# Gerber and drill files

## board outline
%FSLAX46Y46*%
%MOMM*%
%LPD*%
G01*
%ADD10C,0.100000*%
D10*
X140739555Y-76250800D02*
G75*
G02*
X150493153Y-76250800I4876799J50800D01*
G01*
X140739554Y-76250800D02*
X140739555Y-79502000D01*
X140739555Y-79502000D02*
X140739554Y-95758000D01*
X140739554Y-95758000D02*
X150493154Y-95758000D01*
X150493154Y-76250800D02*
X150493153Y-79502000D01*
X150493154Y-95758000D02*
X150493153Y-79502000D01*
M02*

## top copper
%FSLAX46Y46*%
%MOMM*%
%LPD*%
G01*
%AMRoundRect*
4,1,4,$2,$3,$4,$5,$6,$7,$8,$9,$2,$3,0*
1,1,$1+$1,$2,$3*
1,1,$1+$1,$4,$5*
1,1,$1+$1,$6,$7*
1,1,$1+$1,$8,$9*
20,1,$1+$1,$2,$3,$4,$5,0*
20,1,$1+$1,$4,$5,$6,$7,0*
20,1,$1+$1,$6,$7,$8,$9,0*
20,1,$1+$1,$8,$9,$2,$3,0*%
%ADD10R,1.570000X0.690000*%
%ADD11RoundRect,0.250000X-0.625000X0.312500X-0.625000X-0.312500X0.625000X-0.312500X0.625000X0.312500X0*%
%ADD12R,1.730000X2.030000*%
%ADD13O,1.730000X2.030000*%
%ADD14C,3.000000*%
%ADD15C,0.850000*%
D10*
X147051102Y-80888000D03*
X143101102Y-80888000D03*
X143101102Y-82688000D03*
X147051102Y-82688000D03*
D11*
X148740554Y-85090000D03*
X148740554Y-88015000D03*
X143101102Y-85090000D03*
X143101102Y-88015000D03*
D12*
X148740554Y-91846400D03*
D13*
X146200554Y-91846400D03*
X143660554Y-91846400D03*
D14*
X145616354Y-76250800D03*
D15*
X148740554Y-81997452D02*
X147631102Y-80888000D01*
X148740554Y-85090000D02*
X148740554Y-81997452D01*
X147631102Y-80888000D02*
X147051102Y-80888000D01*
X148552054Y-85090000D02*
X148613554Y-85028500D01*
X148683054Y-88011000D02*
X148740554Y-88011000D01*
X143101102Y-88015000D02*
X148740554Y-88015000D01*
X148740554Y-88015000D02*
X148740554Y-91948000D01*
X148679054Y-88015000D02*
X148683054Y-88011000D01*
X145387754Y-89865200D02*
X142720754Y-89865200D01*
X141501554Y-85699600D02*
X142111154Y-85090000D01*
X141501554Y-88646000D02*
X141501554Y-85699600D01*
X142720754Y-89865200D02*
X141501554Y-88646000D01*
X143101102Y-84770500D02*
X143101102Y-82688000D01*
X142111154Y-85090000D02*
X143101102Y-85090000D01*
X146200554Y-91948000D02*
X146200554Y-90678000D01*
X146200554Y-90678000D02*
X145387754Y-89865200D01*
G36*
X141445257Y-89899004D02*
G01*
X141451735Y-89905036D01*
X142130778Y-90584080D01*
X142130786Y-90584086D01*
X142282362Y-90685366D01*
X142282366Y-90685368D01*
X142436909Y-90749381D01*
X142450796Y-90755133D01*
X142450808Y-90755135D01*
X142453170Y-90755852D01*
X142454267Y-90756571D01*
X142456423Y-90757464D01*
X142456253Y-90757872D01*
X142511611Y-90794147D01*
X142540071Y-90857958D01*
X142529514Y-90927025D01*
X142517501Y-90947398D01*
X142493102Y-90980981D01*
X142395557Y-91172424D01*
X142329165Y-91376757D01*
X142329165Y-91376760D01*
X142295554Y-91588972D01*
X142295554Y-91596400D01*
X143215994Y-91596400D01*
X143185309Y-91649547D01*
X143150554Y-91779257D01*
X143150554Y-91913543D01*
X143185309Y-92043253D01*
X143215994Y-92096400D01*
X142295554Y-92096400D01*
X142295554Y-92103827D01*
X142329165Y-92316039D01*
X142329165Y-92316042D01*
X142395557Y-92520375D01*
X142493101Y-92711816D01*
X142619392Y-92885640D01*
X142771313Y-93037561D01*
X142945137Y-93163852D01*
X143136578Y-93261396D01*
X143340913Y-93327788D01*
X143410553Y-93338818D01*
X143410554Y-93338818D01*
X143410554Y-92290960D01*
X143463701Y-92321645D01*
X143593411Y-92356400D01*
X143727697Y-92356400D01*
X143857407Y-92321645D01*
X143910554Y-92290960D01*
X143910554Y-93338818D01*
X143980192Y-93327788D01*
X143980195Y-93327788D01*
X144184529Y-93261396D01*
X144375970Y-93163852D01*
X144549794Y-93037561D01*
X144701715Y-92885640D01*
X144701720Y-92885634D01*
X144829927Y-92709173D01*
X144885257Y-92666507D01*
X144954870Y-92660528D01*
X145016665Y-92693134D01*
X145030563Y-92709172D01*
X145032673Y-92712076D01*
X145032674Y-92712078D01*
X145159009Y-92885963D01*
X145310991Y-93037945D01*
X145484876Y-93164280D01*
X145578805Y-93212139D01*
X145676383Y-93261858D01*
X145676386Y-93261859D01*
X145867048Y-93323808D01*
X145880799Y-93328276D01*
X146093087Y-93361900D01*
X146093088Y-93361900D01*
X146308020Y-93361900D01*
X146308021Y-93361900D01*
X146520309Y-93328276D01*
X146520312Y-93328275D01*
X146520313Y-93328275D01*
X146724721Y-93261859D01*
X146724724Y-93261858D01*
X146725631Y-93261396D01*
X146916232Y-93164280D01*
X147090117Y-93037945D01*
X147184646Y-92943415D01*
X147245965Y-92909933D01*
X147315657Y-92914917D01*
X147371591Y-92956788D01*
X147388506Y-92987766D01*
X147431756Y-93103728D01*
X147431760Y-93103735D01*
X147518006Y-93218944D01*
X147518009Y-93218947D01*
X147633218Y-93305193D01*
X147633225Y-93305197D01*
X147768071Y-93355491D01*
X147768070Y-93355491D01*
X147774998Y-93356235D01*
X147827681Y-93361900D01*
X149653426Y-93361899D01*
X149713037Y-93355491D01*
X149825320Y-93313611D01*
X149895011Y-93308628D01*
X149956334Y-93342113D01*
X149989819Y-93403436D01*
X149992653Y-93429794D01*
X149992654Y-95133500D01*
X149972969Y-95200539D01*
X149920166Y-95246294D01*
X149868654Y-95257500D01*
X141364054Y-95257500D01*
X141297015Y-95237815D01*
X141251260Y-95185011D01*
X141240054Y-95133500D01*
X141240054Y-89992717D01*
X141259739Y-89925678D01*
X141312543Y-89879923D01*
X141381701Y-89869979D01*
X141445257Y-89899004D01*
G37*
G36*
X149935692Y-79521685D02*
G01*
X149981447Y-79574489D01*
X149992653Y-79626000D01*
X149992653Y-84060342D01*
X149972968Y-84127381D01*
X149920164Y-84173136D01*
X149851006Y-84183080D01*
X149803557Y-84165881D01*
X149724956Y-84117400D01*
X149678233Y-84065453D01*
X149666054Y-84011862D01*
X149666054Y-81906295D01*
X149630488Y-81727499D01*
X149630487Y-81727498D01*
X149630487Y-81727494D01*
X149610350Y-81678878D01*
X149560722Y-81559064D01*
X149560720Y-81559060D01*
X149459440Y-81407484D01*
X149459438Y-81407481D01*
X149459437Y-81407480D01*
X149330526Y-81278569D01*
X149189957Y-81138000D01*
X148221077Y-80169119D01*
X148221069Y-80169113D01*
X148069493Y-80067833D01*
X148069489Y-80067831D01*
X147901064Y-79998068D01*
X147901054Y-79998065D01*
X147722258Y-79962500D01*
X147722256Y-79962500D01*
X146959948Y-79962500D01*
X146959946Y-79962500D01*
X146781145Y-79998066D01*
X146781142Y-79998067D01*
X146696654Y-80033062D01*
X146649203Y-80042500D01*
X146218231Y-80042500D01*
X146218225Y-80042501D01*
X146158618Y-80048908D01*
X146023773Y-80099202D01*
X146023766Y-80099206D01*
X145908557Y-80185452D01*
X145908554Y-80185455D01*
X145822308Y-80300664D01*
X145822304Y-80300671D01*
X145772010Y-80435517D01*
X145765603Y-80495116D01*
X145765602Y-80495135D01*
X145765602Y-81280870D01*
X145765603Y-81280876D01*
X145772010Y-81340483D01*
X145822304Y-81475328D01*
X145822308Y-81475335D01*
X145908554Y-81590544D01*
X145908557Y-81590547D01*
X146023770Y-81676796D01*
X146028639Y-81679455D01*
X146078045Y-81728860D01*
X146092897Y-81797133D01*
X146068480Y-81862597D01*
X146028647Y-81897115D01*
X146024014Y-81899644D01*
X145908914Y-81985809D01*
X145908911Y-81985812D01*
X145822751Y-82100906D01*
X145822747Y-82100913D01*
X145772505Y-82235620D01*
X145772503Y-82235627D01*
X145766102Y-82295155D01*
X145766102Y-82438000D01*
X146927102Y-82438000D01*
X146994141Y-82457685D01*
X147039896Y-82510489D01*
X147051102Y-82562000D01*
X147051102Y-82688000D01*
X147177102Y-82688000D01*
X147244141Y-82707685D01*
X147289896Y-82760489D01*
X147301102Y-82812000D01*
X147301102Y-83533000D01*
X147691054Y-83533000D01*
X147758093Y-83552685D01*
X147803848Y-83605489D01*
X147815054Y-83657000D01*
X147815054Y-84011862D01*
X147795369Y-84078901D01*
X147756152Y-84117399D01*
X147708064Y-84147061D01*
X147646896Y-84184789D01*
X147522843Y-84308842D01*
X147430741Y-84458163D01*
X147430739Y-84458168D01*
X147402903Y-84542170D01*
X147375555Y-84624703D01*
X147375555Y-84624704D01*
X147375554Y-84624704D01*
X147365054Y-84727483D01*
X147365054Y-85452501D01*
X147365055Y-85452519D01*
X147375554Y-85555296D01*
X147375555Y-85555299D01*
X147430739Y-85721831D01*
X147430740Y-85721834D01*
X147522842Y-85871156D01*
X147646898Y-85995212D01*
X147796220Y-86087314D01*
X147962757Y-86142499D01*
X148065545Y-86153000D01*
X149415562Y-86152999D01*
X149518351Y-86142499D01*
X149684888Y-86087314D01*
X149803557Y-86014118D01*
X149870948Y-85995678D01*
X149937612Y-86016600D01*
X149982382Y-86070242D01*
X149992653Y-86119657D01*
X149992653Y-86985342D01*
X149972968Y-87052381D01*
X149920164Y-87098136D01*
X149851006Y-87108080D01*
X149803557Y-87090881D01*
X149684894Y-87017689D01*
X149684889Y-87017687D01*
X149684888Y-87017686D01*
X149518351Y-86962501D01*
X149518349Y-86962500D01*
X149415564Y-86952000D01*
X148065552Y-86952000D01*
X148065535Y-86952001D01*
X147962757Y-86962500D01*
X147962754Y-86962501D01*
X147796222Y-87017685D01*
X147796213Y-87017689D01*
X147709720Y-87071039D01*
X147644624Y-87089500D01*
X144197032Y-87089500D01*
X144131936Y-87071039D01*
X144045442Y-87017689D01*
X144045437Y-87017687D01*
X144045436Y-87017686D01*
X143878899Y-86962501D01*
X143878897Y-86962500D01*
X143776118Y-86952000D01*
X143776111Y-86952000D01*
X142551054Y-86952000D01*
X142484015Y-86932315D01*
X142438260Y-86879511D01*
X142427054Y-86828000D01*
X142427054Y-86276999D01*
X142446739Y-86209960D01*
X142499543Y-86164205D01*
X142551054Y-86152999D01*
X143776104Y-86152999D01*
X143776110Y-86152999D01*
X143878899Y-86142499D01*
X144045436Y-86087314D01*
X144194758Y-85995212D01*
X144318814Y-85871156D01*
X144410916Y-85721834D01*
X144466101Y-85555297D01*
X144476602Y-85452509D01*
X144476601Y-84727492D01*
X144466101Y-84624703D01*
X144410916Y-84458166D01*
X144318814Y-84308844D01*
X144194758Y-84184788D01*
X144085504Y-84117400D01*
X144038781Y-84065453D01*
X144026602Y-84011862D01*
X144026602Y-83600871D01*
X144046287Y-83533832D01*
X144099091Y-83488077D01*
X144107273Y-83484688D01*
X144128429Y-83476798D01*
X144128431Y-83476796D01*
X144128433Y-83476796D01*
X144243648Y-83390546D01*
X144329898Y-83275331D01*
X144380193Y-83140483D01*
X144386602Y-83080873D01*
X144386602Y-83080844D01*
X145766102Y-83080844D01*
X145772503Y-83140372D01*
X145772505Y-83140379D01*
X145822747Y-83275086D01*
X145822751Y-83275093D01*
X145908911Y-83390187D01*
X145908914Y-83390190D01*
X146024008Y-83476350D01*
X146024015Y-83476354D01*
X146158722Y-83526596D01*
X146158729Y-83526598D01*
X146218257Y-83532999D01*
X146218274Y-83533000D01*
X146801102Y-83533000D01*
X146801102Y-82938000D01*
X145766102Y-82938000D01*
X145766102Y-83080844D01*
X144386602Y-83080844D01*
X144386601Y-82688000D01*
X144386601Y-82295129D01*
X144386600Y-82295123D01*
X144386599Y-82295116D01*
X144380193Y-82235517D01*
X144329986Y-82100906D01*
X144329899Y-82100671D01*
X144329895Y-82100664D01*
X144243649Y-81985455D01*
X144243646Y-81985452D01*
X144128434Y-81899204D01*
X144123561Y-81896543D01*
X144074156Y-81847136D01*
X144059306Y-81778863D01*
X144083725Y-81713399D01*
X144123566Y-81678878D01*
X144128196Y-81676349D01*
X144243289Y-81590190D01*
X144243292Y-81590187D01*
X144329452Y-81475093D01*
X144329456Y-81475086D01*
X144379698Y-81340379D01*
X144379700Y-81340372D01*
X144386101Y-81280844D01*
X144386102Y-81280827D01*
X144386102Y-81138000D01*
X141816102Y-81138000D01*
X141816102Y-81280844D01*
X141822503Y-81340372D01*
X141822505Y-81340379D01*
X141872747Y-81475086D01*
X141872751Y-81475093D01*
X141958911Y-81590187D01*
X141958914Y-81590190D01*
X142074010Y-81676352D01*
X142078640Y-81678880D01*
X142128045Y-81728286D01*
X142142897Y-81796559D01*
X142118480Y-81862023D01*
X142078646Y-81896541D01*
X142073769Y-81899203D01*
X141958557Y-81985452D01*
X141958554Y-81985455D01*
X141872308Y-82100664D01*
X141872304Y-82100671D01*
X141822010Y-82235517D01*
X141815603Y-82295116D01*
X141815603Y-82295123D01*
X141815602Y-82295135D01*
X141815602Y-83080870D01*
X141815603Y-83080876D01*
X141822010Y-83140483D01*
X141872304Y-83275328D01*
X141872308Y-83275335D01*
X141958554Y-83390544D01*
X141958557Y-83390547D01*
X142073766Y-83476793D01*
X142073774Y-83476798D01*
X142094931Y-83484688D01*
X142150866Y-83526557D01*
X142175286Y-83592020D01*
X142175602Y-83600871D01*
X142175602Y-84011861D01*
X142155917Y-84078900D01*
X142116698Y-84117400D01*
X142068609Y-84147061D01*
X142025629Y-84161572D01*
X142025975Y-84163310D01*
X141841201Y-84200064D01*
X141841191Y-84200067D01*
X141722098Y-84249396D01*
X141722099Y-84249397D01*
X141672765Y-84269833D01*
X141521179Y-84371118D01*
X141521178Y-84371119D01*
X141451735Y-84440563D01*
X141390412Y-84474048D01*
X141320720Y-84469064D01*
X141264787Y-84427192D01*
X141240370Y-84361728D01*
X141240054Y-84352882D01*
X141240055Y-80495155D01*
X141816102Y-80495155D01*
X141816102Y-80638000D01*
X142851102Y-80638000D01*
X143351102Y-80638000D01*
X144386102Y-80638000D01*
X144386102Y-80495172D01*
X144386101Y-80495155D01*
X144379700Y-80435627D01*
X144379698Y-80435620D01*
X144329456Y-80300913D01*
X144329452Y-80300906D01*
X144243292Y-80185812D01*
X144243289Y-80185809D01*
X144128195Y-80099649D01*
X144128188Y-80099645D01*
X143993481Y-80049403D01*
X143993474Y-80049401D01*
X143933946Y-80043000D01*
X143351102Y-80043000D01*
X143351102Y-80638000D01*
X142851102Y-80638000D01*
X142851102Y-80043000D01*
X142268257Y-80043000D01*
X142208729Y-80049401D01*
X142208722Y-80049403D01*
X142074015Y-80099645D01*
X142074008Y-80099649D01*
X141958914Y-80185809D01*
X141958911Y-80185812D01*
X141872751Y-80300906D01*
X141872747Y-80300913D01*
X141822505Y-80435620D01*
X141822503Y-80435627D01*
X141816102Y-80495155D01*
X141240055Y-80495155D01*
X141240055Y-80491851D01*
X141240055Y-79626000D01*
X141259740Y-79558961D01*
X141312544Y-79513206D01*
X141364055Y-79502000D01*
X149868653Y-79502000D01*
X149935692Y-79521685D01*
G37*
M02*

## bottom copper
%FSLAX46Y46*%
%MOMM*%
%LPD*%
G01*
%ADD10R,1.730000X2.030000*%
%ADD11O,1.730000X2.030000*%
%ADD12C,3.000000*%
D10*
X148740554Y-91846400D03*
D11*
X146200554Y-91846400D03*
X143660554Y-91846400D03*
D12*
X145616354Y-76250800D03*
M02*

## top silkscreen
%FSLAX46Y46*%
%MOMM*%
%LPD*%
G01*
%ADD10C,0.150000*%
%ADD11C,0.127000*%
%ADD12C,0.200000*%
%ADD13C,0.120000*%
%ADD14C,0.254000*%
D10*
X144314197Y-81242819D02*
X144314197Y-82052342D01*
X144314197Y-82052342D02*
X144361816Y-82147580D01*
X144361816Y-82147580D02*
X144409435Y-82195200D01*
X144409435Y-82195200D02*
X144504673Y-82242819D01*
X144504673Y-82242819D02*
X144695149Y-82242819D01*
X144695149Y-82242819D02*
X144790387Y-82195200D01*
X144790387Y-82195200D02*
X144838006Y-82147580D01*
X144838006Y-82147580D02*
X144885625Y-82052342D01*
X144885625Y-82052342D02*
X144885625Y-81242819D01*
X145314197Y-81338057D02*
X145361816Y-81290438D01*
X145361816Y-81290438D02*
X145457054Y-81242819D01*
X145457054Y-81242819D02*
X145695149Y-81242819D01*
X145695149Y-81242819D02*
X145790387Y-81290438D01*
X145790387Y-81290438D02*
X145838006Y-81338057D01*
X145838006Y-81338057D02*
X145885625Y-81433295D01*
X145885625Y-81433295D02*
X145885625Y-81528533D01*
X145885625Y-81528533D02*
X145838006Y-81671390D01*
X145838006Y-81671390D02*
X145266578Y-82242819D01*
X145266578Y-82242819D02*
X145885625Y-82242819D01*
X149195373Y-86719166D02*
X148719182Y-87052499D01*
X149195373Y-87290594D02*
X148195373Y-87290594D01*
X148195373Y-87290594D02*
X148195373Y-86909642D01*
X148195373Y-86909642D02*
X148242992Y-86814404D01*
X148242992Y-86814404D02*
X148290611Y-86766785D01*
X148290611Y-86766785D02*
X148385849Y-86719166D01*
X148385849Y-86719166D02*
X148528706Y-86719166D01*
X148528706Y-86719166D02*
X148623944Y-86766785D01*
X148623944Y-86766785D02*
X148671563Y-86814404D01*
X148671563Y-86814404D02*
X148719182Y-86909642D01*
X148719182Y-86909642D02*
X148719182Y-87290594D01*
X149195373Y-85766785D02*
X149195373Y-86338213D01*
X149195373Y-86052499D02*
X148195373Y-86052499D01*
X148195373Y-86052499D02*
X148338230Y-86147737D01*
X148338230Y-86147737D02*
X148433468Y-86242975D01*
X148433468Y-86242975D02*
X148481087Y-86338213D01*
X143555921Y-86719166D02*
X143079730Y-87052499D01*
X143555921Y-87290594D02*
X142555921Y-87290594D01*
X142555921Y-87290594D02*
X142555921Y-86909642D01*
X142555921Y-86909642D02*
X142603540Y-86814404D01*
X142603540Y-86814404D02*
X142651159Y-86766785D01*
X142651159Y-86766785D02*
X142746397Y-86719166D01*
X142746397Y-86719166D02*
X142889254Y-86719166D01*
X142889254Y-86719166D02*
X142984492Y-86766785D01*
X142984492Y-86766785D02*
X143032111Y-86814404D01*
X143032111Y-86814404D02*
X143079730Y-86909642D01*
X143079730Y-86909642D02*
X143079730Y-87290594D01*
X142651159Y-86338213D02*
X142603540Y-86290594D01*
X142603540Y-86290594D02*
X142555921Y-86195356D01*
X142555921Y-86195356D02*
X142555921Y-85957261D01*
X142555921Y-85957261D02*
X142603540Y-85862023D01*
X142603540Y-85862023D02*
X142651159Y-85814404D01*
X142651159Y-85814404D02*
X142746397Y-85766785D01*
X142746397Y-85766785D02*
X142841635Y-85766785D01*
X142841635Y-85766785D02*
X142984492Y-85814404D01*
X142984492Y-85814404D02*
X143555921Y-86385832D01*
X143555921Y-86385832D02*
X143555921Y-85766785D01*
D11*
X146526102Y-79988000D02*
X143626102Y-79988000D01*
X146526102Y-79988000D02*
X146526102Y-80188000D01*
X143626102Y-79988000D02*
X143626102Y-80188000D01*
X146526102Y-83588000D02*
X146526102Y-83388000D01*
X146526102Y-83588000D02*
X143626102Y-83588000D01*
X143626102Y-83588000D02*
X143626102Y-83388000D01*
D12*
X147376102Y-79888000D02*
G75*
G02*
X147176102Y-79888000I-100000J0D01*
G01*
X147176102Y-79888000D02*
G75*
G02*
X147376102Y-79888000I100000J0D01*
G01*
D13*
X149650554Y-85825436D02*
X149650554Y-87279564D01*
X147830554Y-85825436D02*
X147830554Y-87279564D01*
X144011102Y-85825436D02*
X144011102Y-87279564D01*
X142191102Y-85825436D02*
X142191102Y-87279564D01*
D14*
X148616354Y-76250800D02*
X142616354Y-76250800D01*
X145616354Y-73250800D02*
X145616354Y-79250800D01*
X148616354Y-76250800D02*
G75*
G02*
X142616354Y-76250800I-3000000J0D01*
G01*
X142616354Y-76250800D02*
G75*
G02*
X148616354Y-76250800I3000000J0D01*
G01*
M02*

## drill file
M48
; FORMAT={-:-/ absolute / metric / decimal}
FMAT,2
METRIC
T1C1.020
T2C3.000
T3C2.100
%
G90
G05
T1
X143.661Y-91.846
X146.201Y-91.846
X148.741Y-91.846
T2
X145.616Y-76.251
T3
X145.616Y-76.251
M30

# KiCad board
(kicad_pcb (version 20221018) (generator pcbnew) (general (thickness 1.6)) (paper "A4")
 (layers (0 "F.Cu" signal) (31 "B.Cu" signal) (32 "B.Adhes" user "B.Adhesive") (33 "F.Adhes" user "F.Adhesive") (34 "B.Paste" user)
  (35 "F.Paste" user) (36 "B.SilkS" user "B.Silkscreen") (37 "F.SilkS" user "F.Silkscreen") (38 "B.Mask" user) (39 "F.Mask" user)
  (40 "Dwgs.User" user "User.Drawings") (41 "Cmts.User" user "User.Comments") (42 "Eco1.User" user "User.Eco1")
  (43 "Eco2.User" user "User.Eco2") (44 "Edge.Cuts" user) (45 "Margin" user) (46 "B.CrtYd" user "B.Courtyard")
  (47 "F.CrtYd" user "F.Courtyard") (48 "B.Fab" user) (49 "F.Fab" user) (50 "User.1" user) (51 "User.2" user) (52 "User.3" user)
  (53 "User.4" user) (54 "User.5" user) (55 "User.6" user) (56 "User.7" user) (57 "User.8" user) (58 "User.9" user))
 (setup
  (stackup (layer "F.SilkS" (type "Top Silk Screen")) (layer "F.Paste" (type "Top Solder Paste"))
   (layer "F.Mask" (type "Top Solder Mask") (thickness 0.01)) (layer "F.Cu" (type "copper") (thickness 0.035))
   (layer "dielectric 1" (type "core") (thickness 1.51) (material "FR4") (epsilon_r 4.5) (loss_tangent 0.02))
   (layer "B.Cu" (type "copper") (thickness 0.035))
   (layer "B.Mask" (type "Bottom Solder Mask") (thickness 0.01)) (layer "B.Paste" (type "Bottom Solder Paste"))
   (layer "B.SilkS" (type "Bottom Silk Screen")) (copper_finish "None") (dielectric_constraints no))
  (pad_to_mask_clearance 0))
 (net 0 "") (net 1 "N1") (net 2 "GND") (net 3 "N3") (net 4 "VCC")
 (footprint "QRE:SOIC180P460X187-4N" (layer "F.Cu") (at 145.076102 81.788 -90)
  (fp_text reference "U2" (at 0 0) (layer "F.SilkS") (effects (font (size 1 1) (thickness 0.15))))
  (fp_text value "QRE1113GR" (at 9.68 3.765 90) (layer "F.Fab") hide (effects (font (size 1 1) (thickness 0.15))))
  (fp_line (start -1.8 -1.45) (end -1.8 1.45) (stroke (width 0.127) (type solid)) (layer "F.SilkS"))
  (fp_line (start -1.8 -1.45) (end -1.6 -1.45) (stroke (width 0.127) (type solid)) (layer "F.SilkS"))
  (fp_line (start -1.8 1.45) (end -1.6 1.45) (stroke (width 0.127) (type solid)) (layer "F.SilkS"))
  (fp_line (start 1.8 -1.45) (end 1.6 -1.45) (stroke (width 0.127) (type solid)) (layer "F.SilkS"))
  (fp_line (start 1.8 -1.45) (end 1.8 1.45) (stroke (width 0.127) (type solid)) (layer "F.SilkS"))
  (fp_line (start 1.8 1.45) (end 1.6 1.45) (stroke (width 0.127) (type solid)) (layer "F.SilkS"))
  (fp_circle (center -1.9 -2.2) (end -1.8 -2.2) (stroke (width 0.2) (type solid)) (fill none) (layer "F.SilkS"))
  (pad "1" smd rect (at -0.9 -1.975 270) (size 0.69 1.57) (layers "F.Cu" "F.Paste" "F.Mask") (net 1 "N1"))
  (pad "2" smd rect (at -0.9 1.975 270) (size 0.69 1.57) (layers "F.Cu" "F.Paste" "F.Mask") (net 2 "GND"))
  (pad "3" smd rect (at 0.9 1.975 270) (size 0.69 1.57) (layers "F.Cu" "F.Paste" "F.Mask") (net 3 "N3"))
  (pad "4" smd rect (at 0.9 -1.975 270) (size 0.69 1.57) (layers "F.Cu" "F.Paste" "F.Mask") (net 2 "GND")))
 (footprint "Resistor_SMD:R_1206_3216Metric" (layer "F.Cu") (at 148.740554 86.5525 -90)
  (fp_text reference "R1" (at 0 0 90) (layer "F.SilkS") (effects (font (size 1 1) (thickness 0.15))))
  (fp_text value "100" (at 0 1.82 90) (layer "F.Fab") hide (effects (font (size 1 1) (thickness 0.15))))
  (fp_line (start -0.727064 -0.91) (end 0.727064 -0.91) (stroke (width 0.12) (type solid)) (layer "F.SilkS"))
  (fp_line (start -0.727064 0.91) (end 0.727064 0.91) (stroke (width 0.12) (type solid)) (layer "F.SilkS"))
  (pad "1" smd roundrect (at -1.4625 0 270) (size 1.125 1.75) (layers "F.Cu" "F.Paste" "F.Mask") (roundrect_rratio 0.222222) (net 1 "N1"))
  (pad "2" smd roundrect (at 1.4625 0 270) (size 1.125 1.75) (layers "F.Cu" "F.Paste" "F.Mask") (roundrect_rratio 0.222222) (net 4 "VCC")))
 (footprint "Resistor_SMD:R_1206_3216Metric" (layer "F.Cu") (at 143.101102 86.5525 -90)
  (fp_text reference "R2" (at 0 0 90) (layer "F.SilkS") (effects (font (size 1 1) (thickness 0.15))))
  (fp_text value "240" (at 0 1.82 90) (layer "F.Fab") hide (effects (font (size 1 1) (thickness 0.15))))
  (fp_line (start -0.727064 -0.91) (end 0.727064 -0.91) (stroke (width 0.12) (type solid)) (layer "F.SilkS"))
  (fp_line (start -0.727064 0.91) (end 0.727064 0.91) (stroke (width 0.12) (type solid)) (layer "F.SilkS"))
  (pad "1" smd roundrect (at -1.4625 0 270) (size 1.125 1.75) (layers "F.Cu" "F.Paste" "F.Mask") (roundrect_rratio 0.222222) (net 3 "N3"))
  (pad "2" smd roundrect (at 1.4625 0 270) (size 1.125 1.75) (layers "F.Cu" "F.Paste" "F.Mask") (roundrect_rratio 0.222222) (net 4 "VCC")))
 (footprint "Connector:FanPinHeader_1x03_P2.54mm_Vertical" (layer "B.Cu") (at 148.740554 91.8464 180)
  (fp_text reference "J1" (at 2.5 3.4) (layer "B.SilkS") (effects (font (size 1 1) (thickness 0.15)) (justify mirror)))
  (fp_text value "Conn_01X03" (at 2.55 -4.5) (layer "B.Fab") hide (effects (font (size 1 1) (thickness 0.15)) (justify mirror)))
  (pad "1" thru_hole rect (at 0 0 90) (size 2.03 1.73) (drill 1.02) (layers "*.Cu" "*.Mask") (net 4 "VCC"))
  (pad "2" thru_hole oval (at 2.54 0 90) (size 2.03 1.73) (drill 1.02) (layers "*.Cu" "*.Mask") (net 3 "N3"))
  (pad "3" thru_hole oval (at 5.08 0 90) (size 2.03 1.73) (drill 1.02) (layers "*.Cu" "*.Mask") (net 2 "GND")))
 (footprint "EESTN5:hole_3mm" (layer "B.Cu") (at 145.616354 76.2508 180)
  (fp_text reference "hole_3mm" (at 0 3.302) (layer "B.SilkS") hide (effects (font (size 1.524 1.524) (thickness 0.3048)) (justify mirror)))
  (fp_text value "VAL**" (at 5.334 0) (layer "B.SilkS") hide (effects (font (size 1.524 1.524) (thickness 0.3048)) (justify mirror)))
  (fp_line (start -3 0) (end 3 0) (stroke (width 0.254) (type solid)) (layer "F.SilkS"))
  (fp_line (start 0 3) (end 0 -3) (stroke (width 0.254) (type solid)) (layer "F.SilkS"))
  (fp_circle (center 0 0) (end 3 0) (stroke (width 0.254) (type solid)) (fill none) (layer "F.SilkS"))
  (pad "1" thru_hole circle (at 0 0 180) (size 3 3) (drill 3) (layers "*.Cu" "B.SilkS")))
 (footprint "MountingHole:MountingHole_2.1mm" (layer "B.Cu") (at 145.616354 76.2508 180)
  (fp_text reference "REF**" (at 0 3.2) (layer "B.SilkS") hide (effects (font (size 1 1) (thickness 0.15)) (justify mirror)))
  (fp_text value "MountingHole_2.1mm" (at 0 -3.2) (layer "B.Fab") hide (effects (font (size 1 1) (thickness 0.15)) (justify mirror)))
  (pad "" np_thru_hole circle (at 0 0 180) (size 2.1 2.1) (drill 2.1) (layers "*.Cu" "*.Mask")))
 (gr_arc (start 140.739555 76.2508) (mid 145.616354 71.322936) (end 150.493153 76.2508) (stroke (width 0.1) (type default))
  (layer "Edge.Cuts"))
 (gr_line (start 140.739554 76.2508) (end 140.739555 79.502) (stroke (width 0.1) (type default)) (layer "Edge.Cuts"))
 (gr_line (start 140.739555 79.502) (end 140.739554 95.758) (stroke (width 0.1) (type default)) (layer "Edge.Cuts"))
 (gr_line (start 140.739554 95.758) (end 150.493154 95.758) (stroke (width 0.1) (type default)) (layer "Edge.Cuts"))
 (gr_line (start 150.493154 76.2508) (end 150.493153 79.502) (stroke (width 0.1) (type default)) (layer "Edge.Cuts"))
 (gr_line (start 150.493154 95.758) (end 150.493153 79.502) (stroke (width 0.1) (type default)) (layer "Edge.Cuts"))
 (segment (start 148.740554 81.997452) (end 147.631102 80.888) (width 0.85) (layer "F.Cu") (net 1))
 (segment (start 148.740554 85.09) (end 148.740554 81.997452) (width 0.85) (layer "F.Cu") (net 1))
 (segment (start 147.631102 80.888) (end 147.051102 80.888) (width 0.85) (layer "F.Cu") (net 1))
 (segment (start 148.552054 85.09) (end 148.613554 85.0285) (width 0.85) (layer "F.Cu") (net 1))
 (segment (start 148.683054 88.011) (end 148.740554 88.011) (width 0.85) (layer "F.Cu") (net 4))
 (segment (start 143.101102 88.015) (end 148.740554 88.015) (width 0.85) (layer "F.Cu") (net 4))
 (segment (start 148.740554 88.015) (end 148.740554 91.948) (width 0.85) (layer "F.Cu") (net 4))
 (segment (start 148.679054 88.015) (end 148.683054 88.011) (width 0.85) (layer "F.Cu") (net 4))
 (segment (start 145.387754 89.8652) (end 142.720754 89.8652) (width 0.85) (layer "F.Cu") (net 3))
 (segment (start 141.501554 85.6996) (end 142.111154 85.09) (width 0.85) (layer "F.Cu") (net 3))
 (segment (start 141.501554 88.646) (end 141.501554 85.6996) (width 0.85) (layer "F.Cu") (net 3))
 (segment (start 142.720754 89.8652) (end 141.501554 88.646) (width 0.85) (layer "F.Cu") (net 3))
 (segment (start 143.101102 84.7705) (end 143.101102 82.688) (width 0.85) (layer "F.Cu") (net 3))
 (segment (start 142.111154 85.09) (end 143.101102 85.09) (width 0.85) (layer "F.Cu") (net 3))
 (segment (start 146.200554 91.948) (end 146.200554 90.678) (width 0.85) (layer "F.Cu") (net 3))
 (segment (start 146.200554 90.678) (end 145.387754 89.8652) (width 0.85) (layer "F.Cu") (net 3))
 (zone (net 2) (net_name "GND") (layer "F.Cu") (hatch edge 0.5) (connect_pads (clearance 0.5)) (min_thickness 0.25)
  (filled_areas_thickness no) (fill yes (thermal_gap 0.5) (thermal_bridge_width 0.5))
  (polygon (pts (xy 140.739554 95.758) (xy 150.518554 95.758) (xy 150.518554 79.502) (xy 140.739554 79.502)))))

